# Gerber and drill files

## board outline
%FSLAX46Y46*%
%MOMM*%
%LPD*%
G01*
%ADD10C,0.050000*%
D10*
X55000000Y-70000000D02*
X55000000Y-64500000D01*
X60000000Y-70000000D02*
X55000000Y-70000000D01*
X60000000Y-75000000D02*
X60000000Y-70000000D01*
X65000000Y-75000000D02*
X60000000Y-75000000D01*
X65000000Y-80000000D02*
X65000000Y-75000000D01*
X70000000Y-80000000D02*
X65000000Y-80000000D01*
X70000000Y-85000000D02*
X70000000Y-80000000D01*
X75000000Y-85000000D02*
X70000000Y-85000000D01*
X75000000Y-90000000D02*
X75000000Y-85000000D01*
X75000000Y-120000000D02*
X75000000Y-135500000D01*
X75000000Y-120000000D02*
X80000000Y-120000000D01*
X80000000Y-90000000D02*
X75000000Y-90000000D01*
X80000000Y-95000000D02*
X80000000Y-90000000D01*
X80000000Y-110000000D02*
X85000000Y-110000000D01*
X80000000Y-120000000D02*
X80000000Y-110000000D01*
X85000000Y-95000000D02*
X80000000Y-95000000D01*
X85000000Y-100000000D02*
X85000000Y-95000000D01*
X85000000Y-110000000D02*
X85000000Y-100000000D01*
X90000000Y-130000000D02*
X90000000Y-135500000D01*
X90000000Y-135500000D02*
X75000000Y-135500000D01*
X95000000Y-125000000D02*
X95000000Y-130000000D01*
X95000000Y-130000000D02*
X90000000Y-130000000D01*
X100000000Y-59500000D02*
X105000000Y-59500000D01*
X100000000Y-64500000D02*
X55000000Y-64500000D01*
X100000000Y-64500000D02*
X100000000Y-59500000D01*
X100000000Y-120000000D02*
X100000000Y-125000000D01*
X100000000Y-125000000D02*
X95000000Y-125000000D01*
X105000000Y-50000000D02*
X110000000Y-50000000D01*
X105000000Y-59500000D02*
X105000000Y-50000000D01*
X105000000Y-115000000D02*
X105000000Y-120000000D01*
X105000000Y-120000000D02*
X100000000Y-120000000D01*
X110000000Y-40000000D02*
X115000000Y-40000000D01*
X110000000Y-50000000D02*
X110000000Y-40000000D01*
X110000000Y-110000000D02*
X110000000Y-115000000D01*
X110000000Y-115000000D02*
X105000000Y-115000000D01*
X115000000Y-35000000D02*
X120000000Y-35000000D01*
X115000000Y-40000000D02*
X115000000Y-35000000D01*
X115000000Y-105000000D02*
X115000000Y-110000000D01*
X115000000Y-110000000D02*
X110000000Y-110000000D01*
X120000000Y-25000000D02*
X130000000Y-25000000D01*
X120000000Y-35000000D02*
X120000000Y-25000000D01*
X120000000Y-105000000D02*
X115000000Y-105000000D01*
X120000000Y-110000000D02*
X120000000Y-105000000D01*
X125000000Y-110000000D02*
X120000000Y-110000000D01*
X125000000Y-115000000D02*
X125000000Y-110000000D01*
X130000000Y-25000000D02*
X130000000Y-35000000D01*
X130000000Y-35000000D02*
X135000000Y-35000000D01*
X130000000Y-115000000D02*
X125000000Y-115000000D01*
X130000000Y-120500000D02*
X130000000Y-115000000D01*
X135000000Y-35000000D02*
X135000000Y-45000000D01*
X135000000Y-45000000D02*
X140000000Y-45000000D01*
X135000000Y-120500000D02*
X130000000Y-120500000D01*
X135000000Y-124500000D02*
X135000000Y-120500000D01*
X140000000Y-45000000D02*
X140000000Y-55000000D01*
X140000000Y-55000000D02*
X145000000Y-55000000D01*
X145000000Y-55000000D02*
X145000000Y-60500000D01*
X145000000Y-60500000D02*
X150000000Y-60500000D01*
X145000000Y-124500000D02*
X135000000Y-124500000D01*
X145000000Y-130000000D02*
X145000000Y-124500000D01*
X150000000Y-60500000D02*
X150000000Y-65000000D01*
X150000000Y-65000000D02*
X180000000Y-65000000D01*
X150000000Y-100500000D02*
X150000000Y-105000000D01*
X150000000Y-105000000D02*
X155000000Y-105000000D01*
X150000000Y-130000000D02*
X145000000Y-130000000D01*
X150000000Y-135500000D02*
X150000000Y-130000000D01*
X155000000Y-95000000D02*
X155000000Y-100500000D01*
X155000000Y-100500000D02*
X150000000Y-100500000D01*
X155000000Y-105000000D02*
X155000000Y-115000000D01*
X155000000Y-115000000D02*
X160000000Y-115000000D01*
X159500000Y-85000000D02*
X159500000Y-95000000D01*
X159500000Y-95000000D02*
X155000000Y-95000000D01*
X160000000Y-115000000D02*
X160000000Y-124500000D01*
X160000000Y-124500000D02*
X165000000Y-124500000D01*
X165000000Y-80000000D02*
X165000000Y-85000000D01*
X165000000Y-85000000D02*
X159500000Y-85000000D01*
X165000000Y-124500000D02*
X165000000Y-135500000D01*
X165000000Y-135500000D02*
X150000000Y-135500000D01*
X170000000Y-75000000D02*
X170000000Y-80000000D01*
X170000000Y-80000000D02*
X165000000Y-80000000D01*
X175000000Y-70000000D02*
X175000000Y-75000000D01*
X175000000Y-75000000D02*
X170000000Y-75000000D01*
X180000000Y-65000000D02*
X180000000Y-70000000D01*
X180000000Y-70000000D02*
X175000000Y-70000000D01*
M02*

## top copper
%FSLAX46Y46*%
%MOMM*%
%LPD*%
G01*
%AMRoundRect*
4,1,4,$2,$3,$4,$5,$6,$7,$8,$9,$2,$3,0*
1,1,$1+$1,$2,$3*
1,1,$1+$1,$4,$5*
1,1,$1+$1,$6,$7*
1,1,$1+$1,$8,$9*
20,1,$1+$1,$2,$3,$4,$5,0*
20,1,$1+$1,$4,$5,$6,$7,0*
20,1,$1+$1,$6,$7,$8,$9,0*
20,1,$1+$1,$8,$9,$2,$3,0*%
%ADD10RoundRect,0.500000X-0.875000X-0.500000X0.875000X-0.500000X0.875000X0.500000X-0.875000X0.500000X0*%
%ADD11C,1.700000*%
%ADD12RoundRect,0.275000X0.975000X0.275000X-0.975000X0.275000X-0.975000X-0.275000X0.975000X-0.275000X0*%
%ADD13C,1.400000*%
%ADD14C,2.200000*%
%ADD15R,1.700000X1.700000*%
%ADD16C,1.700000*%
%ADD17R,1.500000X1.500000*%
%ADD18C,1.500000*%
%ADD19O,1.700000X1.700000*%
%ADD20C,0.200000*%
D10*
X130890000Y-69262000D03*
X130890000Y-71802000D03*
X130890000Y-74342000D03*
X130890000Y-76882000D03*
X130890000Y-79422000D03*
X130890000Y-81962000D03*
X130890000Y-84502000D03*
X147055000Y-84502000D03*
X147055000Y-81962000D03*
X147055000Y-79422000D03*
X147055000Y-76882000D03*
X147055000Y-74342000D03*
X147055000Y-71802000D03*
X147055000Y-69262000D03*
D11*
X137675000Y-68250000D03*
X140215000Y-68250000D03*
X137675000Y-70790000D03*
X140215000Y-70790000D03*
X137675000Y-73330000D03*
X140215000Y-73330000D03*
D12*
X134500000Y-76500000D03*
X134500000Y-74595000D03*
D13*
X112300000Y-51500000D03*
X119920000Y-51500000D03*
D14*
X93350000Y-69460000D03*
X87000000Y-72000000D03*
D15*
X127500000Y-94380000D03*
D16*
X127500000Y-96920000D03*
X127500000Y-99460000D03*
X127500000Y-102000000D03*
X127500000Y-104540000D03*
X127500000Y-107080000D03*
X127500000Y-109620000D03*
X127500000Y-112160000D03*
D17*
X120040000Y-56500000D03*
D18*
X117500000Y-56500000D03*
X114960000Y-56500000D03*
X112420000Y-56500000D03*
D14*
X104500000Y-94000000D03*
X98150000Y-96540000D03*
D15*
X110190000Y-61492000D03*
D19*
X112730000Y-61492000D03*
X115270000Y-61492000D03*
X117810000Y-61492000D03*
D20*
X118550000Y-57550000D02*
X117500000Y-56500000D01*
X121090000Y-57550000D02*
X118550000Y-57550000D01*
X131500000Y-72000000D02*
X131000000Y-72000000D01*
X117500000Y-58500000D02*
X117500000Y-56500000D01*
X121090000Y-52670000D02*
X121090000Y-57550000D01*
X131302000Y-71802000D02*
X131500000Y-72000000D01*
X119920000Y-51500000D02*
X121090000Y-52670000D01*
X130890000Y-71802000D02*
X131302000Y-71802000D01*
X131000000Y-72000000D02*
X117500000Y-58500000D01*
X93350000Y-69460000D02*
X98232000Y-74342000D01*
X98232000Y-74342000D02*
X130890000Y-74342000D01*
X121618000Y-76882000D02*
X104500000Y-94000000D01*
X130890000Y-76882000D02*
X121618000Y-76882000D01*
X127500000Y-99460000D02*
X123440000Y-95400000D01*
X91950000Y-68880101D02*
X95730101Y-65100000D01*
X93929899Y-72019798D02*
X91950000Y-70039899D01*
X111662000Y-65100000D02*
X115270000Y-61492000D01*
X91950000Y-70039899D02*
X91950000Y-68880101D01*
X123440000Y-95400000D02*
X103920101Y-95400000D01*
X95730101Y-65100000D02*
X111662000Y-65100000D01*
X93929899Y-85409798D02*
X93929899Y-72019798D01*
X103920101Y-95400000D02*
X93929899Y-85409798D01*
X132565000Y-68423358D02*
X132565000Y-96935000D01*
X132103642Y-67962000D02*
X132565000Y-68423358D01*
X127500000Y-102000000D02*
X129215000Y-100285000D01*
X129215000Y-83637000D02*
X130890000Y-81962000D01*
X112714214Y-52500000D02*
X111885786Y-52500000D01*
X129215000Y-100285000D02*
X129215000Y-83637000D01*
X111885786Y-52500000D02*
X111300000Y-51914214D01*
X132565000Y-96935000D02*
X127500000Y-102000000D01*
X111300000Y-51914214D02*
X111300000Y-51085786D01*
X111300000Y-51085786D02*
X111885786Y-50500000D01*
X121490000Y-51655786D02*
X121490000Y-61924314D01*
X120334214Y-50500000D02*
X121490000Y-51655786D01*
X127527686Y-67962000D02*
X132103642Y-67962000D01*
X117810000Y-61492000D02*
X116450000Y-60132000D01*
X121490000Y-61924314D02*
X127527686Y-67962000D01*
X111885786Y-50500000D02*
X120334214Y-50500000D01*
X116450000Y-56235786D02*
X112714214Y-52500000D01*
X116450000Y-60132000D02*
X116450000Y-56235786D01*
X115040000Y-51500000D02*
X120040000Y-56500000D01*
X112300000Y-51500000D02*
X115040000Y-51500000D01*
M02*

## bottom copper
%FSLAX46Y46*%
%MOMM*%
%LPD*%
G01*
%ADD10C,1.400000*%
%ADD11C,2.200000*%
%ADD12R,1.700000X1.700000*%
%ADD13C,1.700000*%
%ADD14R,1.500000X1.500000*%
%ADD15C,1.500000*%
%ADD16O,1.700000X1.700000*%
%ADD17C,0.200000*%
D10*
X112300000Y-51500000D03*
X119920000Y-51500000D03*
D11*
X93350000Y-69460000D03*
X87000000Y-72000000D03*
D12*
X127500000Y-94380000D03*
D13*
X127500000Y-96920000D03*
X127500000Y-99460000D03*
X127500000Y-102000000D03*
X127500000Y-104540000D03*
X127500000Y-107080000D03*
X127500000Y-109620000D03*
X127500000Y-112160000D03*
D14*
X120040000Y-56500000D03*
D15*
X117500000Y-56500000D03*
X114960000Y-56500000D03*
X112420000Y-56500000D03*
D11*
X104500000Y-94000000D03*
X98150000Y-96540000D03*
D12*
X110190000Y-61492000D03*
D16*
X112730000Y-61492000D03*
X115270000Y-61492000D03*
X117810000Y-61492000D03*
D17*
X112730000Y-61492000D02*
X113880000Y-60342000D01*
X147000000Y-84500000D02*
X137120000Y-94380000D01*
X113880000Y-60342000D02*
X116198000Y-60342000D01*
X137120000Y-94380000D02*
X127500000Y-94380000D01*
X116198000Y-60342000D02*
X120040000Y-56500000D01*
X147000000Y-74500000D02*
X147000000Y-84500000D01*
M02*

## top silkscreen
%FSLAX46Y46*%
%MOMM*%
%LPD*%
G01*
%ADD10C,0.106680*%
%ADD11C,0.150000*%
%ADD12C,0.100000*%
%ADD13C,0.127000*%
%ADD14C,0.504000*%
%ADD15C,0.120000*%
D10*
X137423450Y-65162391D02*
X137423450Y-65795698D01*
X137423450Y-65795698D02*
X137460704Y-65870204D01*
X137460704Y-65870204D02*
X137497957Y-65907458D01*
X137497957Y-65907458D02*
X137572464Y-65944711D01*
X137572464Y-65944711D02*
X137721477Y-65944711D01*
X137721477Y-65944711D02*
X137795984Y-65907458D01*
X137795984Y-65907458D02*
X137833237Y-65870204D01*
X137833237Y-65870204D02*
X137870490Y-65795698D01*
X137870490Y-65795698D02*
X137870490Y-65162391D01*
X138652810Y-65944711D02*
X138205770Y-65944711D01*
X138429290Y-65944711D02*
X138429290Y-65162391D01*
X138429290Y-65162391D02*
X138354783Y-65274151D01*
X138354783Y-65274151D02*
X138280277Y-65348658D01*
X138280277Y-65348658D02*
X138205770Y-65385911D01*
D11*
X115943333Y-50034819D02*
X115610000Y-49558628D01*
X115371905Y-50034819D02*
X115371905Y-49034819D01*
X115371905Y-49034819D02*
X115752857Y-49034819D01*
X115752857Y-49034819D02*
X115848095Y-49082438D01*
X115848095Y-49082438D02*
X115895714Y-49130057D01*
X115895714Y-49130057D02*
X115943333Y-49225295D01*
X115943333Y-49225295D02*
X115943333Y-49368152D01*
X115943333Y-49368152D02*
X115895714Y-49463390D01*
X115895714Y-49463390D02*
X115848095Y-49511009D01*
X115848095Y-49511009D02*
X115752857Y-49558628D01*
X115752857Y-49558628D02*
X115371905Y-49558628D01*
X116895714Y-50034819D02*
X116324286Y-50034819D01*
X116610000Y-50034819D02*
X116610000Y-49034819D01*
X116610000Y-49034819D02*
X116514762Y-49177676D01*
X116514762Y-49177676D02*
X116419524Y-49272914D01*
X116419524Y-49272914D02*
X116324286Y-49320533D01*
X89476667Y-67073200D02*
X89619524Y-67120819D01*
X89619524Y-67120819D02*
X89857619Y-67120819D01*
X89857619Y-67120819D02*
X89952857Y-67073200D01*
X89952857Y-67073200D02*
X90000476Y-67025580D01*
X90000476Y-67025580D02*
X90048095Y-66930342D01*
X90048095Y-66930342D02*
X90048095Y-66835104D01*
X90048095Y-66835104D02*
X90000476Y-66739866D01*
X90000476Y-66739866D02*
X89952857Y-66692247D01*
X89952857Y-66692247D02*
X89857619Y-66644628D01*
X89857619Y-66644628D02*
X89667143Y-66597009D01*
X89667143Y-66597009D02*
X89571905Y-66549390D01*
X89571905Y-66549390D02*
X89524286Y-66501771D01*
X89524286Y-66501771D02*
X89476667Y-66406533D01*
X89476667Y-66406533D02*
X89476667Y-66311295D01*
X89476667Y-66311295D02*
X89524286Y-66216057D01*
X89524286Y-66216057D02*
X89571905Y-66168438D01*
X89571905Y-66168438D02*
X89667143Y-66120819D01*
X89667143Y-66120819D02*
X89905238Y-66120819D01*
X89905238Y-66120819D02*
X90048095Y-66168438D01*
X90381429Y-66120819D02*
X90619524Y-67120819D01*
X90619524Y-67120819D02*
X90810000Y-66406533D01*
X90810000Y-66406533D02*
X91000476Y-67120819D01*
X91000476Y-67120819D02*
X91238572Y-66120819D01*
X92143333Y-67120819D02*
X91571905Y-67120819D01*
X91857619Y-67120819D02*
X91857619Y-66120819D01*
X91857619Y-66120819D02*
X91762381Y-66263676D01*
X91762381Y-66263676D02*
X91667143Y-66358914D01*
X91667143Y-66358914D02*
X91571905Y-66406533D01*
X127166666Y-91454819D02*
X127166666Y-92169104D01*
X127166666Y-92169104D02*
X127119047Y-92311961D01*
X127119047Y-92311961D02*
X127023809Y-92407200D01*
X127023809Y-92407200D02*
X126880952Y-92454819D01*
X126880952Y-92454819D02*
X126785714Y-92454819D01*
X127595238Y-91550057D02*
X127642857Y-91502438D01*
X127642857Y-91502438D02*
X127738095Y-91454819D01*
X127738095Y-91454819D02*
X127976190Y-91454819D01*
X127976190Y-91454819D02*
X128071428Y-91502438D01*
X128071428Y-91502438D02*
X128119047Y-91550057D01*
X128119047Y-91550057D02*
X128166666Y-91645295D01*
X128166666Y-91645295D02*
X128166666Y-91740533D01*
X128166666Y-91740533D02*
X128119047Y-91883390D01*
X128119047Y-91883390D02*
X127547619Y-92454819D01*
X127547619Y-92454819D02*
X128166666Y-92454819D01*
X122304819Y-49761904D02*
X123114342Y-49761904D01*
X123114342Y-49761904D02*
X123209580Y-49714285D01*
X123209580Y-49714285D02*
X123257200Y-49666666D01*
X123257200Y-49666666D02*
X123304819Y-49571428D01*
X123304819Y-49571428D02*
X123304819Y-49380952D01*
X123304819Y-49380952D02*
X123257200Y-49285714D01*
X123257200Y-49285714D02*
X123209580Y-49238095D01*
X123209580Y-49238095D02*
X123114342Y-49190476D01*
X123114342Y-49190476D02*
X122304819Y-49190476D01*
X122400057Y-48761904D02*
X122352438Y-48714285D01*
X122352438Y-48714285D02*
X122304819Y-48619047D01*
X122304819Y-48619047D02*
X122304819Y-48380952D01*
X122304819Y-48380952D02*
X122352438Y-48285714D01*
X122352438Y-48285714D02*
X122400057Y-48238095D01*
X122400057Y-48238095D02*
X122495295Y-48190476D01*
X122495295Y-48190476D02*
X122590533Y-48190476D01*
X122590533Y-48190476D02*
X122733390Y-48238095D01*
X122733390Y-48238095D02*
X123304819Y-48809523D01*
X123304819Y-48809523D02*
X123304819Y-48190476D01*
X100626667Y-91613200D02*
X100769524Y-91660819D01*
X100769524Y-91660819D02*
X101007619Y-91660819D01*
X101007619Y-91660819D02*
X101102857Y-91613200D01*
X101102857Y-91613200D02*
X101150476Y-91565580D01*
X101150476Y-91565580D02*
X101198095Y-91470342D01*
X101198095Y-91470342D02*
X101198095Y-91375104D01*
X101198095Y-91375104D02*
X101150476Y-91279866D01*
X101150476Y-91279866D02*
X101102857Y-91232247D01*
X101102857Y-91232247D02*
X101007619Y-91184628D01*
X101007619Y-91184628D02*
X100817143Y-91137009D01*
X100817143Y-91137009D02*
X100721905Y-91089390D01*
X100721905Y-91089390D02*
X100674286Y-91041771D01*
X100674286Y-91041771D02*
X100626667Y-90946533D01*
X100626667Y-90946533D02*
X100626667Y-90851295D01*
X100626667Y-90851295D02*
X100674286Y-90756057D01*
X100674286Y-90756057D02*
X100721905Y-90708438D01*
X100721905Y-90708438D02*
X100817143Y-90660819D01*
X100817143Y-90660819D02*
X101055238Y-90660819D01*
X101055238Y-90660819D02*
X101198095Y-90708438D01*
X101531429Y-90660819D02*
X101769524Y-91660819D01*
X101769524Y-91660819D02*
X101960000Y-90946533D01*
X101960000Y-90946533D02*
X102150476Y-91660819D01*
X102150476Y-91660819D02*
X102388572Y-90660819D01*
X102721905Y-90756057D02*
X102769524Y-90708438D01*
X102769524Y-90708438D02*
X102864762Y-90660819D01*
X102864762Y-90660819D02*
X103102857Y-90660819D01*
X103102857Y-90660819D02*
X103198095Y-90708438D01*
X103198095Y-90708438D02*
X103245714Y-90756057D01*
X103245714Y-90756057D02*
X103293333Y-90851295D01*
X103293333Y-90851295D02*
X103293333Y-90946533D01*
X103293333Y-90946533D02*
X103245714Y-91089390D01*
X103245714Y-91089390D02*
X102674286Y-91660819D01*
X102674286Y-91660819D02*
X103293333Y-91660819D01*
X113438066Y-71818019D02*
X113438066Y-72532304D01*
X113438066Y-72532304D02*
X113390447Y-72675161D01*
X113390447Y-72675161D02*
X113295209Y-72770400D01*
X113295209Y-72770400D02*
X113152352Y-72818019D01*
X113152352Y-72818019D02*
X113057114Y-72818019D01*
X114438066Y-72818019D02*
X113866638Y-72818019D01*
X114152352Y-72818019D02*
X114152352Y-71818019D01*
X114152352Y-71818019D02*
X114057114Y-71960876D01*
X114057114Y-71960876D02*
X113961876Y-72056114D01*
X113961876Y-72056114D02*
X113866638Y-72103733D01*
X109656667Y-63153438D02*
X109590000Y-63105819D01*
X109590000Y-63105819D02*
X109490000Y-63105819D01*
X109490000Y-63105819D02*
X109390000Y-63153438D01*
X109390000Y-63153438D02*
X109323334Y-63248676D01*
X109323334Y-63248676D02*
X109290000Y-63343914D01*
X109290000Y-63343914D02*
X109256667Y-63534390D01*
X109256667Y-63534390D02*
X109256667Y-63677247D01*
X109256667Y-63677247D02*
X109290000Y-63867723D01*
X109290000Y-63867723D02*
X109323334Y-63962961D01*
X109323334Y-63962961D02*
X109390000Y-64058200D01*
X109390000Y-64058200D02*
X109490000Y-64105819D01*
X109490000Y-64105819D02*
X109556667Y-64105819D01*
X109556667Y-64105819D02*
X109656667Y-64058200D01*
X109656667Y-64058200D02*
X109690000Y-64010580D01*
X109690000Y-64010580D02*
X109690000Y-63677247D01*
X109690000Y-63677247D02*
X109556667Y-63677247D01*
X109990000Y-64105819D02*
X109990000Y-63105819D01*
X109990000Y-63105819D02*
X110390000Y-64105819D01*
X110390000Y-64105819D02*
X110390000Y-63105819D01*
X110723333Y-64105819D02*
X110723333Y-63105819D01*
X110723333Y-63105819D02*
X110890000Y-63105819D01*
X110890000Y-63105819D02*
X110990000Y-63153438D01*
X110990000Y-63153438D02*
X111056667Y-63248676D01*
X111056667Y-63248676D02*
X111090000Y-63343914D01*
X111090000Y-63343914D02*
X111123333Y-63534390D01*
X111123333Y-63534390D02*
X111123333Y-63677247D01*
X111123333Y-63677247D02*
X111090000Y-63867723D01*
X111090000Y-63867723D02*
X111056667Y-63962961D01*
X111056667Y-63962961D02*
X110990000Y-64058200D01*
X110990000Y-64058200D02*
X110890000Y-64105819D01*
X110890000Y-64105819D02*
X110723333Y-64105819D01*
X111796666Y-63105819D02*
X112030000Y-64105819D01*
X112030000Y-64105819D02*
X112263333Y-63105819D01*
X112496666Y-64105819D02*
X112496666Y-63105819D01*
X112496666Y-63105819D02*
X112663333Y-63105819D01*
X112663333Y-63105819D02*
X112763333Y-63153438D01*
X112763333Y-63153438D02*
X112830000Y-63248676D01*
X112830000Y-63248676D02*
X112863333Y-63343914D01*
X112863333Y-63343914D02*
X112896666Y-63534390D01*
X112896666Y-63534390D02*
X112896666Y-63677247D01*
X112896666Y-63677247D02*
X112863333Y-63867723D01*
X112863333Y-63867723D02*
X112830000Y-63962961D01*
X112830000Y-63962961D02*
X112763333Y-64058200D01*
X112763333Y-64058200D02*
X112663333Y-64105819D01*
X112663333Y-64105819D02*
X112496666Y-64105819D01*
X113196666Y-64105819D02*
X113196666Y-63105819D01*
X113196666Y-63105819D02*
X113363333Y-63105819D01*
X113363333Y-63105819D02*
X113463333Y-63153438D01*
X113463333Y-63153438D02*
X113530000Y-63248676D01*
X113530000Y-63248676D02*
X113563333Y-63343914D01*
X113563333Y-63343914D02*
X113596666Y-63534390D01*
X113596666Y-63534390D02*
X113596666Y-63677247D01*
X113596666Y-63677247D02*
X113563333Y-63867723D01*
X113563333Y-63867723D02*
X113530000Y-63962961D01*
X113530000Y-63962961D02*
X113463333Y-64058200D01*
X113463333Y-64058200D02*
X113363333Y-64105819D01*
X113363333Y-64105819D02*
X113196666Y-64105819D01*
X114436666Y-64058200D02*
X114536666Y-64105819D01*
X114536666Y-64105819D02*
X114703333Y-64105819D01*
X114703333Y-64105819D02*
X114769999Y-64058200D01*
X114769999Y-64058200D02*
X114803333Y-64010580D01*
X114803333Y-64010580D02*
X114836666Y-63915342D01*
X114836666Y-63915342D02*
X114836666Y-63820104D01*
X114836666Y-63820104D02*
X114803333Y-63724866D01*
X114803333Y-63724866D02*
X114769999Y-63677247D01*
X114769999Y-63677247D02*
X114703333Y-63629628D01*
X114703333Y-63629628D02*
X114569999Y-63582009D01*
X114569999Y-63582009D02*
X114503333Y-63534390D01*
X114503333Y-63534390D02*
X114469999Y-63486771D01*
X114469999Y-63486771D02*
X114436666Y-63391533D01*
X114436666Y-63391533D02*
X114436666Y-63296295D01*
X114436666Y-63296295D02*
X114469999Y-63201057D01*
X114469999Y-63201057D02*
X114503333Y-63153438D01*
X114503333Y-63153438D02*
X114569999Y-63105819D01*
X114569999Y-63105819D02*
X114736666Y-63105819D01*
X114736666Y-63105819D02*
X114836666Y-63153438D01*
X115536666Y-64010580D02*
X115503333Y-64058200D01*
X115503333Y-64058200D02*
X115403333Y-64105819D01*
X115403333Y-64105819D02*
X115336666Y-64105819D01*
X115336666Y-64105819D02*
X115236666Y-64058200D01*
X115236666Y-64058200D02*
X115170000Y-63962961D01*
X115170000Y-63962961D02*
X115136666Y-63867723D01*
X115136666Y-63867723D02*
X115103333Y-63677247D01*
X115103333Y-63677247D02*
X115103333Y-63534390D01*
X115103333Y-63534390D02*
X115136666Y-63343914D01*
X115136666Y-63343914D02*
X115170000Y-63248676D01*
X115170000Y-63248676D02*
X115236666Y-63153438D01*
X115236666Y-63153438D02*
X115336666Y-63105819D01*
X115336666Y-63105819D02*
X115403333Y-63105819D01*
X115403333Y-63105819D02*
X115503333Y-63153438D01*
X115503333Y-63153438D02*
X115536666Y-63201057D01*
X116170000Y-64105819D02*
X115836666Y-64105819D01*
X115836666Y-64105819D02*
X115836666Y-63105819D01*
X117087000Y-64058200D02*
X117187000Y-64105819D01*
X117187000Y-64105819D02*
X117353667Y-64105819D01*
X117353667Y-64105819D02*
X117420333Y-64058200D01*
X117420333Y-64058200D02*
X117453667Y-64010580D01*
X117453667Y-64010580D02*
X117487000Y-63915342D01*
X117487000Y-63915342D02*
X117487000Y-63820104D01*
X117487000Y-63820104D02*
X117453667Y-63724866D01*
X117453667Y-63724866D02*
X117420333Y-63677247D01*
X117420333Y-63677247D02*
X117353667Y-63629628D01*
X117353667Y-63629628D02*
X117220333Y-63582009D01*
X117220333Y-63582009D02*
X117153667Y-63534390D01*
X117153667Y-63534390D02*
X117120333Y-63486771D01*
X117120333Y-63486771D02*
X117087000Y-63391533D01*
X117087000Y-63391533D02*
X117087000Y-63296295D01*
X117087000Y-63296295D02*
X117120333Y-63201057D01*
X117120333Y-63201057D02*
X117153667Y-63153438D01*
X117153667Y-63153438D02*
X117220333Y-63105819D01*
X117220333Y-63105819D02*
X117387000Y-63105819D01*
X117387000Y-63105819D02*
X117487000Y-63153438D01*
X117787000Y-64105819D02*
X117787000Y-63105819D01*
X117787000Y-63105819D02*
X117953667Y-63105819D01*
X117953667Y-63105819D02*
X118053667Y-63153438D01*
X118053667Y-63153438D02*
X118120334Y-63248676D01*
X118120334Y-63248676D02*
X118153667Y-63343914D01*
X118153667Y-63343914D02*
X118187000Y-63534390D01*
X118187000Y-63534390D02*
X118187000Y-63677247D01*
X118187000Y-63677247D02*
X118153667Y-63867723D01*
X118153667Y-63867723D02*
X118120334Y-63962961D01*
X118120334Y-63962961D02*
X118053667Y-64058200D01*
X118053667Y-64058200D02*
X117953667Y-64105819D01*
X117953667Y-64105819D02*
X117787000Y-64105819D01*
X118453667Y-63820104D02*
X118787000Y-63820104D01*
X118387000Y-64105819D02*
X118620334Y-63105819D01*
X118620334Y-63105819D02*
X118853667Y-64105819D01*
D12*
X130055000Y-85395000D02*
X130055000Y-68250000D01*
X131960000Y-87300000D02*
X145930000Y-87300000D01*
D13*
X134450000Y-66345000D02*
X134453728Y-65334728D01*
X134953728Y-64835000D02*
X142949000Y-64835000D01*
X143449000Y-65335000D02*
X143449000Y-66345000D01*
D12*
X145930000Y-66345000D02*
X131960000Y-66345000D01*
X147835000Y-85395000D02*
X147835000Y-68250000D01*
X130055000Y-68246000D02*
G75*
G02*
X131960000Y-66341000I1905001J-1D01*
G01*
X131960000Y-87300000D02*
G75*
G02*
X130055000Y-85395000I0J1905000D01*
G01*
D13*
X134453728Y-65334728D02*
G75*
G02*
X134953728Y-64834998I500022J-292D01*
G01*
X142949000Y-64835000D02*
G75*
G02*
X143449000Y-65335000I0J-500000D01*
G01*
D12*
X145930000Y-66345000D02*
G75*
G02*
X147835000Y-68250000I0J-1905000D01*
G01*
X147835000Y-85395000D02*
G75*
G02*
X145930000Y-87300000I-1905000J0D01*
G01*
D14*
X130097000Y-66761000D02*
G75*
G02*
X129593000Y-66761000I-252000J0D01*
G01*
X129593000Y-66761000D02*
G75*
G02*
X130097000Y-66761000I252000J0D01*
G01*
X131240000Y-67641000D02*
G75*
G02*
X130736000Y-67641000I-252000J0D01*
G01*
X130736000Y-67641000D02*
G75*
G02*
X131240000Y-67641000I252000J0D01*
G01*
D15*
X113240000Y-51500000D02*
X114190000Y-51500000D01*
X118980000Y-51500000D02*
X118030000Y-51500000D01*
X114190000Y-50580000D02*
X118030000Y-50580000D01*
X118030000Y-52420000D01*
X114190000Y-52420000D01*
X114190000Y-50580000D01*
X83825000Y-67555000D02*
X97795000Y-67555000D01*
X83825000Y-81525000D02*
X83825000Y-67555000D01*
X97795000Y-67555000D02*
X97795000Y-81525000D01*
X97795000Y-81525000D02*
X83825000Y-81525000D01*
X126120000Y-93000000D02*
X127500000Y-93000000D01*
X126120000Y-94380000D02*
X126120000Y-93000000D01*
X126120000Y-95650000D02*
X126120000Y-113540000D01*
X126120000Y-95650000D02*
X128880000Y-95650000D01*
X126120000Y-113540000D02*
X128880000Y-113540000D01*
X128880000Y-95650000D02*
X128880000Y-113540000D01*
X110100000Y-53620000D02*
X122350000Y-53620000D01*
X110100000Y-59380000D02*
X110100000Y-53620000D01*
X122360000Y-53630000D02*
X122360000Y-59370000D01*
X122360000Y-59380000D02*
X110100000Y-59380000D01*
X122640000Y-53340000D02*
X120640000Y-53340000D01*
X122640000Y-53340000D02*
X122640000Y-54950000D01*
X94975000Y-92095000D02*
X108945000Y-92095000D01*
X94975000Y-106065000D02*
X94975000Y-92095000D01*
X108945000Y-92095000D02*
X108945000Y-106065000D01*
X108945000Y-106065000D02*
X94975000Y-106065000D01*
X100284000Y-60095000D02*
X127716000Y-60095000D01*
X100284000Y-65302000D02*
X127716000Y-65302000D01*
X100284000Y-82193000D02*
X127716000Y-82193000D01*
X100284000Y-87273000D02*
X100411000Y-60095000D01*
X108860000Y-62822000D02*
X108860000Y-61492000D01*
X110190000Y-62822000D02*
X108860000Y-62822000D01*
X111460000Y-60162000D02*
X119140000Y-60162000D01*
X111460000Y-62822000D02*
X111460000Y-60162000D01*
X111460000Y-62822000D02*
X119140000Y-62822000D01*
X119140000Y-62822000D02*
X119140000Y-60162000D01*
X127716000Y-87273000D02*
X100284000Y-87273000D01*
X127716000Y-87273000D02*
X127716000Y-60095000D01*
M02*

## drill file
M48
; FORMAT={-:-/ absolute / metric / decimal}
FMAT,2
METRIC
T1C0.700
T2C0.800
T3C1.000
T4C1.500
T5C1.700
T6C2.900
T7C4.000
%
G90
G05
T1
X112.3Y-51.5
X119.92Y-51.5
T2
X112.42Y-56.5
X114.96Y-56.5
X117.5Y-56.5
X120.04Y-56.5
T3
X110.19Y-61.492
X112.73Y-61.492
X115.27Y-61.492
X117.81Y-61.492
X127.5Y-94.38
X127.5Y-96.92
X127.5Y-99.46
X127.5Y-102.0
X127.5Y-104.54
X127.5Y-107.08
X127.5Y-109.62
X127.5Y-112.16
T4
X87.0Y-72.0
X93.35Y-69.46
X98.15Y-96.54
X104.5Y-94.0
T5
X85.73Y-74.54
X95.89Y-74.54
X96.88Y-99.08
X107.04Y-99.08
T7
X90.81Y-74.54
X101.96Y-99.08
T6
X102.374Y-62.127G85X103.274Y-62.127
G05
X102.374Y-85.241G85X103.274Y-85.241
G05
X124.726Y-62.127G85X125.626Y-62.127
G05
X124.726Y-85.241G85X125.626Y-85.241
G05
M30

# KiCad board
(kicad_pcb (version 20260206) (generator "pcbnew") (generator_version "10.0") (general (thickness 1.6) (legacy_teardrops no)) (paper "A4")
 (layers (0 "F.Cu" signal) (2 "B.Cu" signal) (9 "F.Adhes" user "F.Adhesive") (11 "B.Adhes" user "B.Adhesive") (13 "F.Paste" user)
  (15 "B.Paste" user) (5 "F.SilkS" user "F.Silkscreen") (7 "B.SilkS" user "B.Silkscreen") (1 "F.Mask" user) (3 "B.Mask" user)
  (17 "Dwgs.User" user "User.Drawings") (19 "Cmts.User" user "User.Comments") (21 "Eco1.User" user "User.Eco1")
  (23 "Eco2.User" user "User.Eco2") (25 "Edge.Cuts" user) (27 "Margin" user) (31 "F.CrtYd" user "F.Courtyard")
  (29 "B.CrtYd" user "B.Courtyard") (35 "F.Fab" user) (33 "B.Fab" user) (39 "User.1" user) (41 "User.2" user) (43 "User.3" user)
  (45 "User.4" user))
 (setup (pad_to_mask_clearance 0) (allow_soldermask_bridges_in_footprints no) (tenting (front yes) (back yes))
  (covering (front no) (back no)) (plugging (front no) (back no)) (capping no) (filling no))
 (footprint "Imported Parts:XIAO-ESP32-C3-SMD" (layer "F.Cu") (at 130.055 87.382)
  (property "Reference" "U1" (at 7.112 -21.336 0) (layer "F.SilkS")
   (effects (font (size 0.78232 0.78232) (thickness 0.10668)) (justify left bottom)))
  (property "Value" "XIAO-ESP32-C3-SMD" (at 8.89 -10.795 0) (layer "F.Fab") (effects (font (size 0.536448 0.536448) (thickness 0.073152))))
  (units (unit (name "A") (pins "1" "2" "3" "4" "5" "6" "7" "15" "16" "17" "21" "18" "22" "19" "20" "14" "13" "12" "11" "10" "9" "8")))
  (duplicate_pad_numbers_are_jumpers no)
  (fp_line (start 0 -1.987) (end 0 -19.132) (stroke (width 0.1) (type solid)) (layer "F.SilkS"))
  (fp_line (start 1.905 -0.082) (end 15.875 -0.082) (stroke (width 0.1) (type solid)) (layer "F.SilkS"))
  (fp_line (start 4.395 -21.037) (end 4.398728 -22.047272) (stroke (width 0.127) (type solid)) (layer "F.SilkS"))
  (fp_line (start 4.898728 -22.547) (end 12.894 -22.547) (stroke (width 0.127) (type solid)) (layer "F.SilkS"))
  (fp_line (start 13.394 -22.047) (end 13.394 -21.037) (stroke (width 0.127) (type solid)) (layer "F.SilkS"))
  (fp_line (start 15.875 -21.037) (end 1.905 -21.037) (stroke (width 0.1) (type solid)) (layer "F.SilkS"))
  (fp_line (start 17.78 -1.987) (end 17.78 -19.132) (stroke (width 0.1) (type solid)) (layer "F.SilkS"))
  (fp_arc (start 0 -19.136) (mid 0.557962 -20.483038) (end 1.905 -21.041) (stroke (width 0.1) (type solid)) (layer "F.SilkS"))
  (fp_arc (start 1.905 -0.082) (mid 0.557962 -0.639962) (end 0 -1.987) (stroke (width 0.1) (type solid)) (layer "F.SilkS"))
  (fp_arc (start 4.398728 -22.047272) (mid 4.545272 -22.40064) (end 4.898728 -22.547) (stroke (width 0.127) (type default))
   (layer "F.SilkS"))
  (fp_arc (start 12.894 -22.547) (mid 13.247553 -22.400553) (end 13.394 -22.047) (stroke (width 0.127) (type default)) (layer "F.SilkS"))
  (fp_arc (start 15.875 -21.037) (mid 17.222038 -20.479038) (end 17.78 -19.132) (stroke (width 0.1) (type solid)) (layer "F.SilkS"))
  (fp_arc (start 17.78 -1.987) (mid 17.222038 -0.639962) (end 15.875 -0.082) (stroke (width 0.1) (type solid)) (layer "F.SilkS"))
  (fp_circle (center -0.21 -20.621) (end -0.21 -20.875) (stroke (width 0.5) (type solid)) (fill yes) (layer "F.SilkS"))
  (fp_circle (center 0.933 -19.741) (end 0.933 -19.995) (stroke (width 0.5) (type solid)) (fill yes) (layer "F.SilkS"))
  (pad "1" smd roundrect (at 0.835 -18.12) (size 2.75 2) (layers "F.Cu" "F.Mask" "F.Paste") (roundrect_rratio 0.25)
   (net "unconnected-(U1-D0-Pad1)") (solder_mask_margin 0.0508) (thermal_bridge_angle 45))
  (pad "2" smd roundrect (at 0.835 -15.58) (size 2.75 2) (layers "F.Cu" "F.Mask" "F.Paste") (roundrect_rratio 0.25) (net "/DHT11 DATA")
   (solder_mask_margin 0.0508) (thermal_bridge_angle 45))
  (pad "3" smd roundrect (at 0.835 -13.04) (size 2.75 2) (layers "F.Cu" "F.Mask" "F.Paste") (roundrect_rratio 0.25) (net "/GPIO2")
   (solder_mask_margin 0.0508) (thermal_bridge_angle 45))
  (pad "4" smd roundrect (at 0.835 -10.5) (size 2.75 2) (layers "F.Cu" "F.Mask" "F.Paste") (roundrect_rratio 0.25) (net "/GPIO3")
   (solder_mask_margin 0.0508) (thermal_bridge_angle 45))
  (pad "5" smd roundrect (at 0.835 -7.96) (size 2.75 2) (layers "F.Cu" "F.Mask" "F.Paste") (roundrect_rratio 0.25) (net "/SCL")
   (solder_mask_margin 0.0508) (thermal_bridge_angle 45))
  (pad "6" smd roundrect (at 0.835 -5.42) (size 2.75 2) (layers "F.Cu" "F.Mask" "F.Paste") (roundrect_rratio 0.25) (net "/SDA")
   (solder_mask_margin 0.0508) (thermal_bridge_angle 45))
  (pad "7" smd roundrect (at 0.835 -2.88) (size 2.75 2) (layers "F.Cu" "F.Mask" "F.Paste") (roundrect_rratio 0.25)
   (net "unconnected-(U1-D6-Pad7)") (solder_mask_margin 0.0508) (thermal_bridge_angle 45))
  (pad "8" smd roundrect (at 17 -2.88) (size 2.75 2) (layers "F.Cu" "F.Mask" "F.Paste") (roundrect_rratio 0.25)
   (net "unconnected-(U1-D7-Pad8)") (solder_mask_margin 0.0508) (thermal_bridge_angle 45))
  (pad "9" smd roundrect (at 17 -5.42) (size 2.75 2) (layers "F.Cu" "F.Mask" "F.Paste") (roundrect_rratio 0.25)
   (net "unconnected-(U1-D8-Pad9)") (solder_mask_margin 0.0508) (thermal_bridge_angle 45))
  (pad "10" smd roundrect (at 17 -7.96) (size 2.75 2) (layers "F.Cu" "F.Mask" "F.Paste") (roundrect_rratio 0.25)
   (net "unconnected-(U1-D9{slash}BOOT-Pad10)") (solder_mask_margin 0.0508) (thermal_bridge_angle 45))
  (pad "11" smd roundrect (at 17 -10.5) (size 2.75 2) (layers "F.Cu" "F.Mask" "F.Paste") (roundrect_rratio 0.25)
   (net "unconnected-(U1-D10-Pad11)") (solder_mask_margin 0.0508) (thermal_bridge_angle 45))
  (pad "12" smd roundrect (at 17 -13.04) (size 2.75 2) (layers "F.Cu" "F.Mask" "F.Paste") (roundrect_rratio 0.25) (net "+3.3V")
   (solder_mask_margin 0.0508) (thermal_bridge_angle 45))
  (pad "13" smd roundrect (at 17 -15.58) (size 2.75 2) (layers "F.Cu" "F.Mask" "F.Paste") (roundrect_rratio 0.25) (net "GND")
   (solder_mask_margin 0.0508) (thermal_bridge_angle 45))
  (pad "14" smd roundrect (at 17 -18.12) (size 2.75 2) (layers "F.Cu" "F.Mask" "F.Paste") (roundrect_rratio 0.25) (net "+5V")
   (solder_mask_margin 0.0508) (thermal_bridge_angle 45))
  (pad "15" smd circle (at 7.62 -19.132) (size 1.7 1.7) (layers "F.Cu" "F.Mask" "F.Paste") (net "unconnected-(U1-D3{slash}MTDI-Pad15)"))
  (pad "16" smd circle (at 10.16 -19.132) (size 1.7 1.7) (layers "F.Cu" "F.Mask" "F.Paste") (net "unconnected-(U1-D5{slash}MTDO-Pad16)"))
  (pad "17" smd circle (at 7.62 -16.592) (size 1.7 1.7) (layers "F.Cu" "F.Mask" "F.Paste") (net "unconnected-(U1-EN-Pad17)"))
  (pad "18" smd circle (at 10.16 -16.592) (size 1.7 1.7) (layers "F.Cu" "F.Mask" "F.Paste") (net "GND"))
  (pad "19" smd circle (at 7.62 -14.052) (size 1.7 1.7) (layers "F.Cu" "F.Mask" "F.Paste") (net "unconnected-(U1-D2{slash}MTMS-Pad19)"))
  (pad "20" smd circle (at 10.16 -14.052) (size 1.7 1.7) (layers "F.Cu" "F.Mask" "F.Paste") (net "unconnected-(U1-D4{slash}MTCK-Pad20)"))
  (pad "21" smd roundrect (at 4.445 -10.882 180) (size 2.5 1.1) (layers "F.Cu" "F.Mask" "F.Paste") (roundrect_rratio 0.25)
   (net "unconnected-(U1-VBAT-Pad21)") (thermal_bridge_angle 45))
  (pad "22" smd roundrect (at 4.445 -12.787 180) (size 2.5 1.1) (layers "F.Cu" "F.Mask" "F.Paste") (roundrect_rratio 0.25)
   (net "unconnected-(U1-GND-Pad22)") (thermal_bridge_angle 45)))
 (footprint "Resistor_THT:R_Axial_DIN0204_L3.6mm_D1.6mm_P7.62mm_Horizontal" (layer "F.Cu") (at 112.3 51.5)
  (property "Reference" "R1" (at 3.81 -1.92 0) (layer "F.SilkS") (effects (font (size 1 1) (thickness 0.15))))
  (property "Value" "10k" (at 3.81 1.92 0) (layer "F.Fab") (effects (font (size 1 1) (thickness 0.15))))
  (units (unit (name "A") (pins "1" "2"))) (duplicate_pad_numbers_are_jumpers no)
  (fp_line (start 0.94 0) (end 1.89 0) (stroke (width 0.12) (type solid)) (layer "F.SilkS"))
  (fp_line (start 6.68 0) (end 5.73 0) (stroke (width 0.12) (type solid)) (layer "F.SilkS"))
  (fp_rect (start 1.89 -0.92) (end 5.73 0.92) (stroke (width 0.12) (type solid)) (fill no) (layer "F.SilkS"))
  (pad "1" thru_hole circle (at 0 0) (size 1.4 1.4) (drill 0.7) (layers "*.Cu" "*.Mask") (remove_unused_layers no) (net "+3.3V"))
  (pad "2" thru_hole circle (at 7.62 0) (size 1.4 1.4) (drill 0.7) (layers "*.Cu" "*.Mask") (remove_unused_layers no) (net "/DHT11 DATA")))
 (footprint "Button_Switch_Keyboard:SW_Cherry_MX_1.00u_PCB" (layer "F.Cu") (at 93.35 69.46)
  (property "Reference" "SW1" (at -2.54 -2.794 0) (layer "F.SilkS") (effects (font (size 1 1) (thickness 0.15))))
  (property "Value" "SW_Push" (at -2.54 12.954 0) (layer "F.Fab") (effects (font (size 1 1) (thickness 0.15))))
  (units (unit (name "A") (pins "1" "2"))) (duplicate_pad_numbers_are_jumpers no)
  (fp_line (start -9.525 -1.905) (end 4.445 -1.905) (stroke (width 0.12) (type solid)) (layer "F.SilkS"))
  (fp_line (start -9.525 12.065) (end -9.525 -1.905) (stroke (width 0.12) (type solid)) (layer "F.SilkS"))
  (fp_line (start 4.445 -1.905) (end 4.445 12.065) (stroke (width 0.12) (type solid)) (layer "F.SilkS"))
  (fp_line (start 4.445 12.065) (end -9.525 12.065) (stroke (width 0.12) (type solid)) (layer "F.SilkS"))
  (pad "" np_thru_hole circle (at -7.62 5.08) (size 1.7 1.7) (drill 1.7) (layers "*.Cu" "*.Mask"))
  (pad "" np_thru_hole circle (at -2.54 5.08) (size 4 4) (drill 4) (layers "*.Cu" "*.Mask"))
  (pad "" np_thru_hole circle (at 2.54 5.08) (size 1.7 1.7) (drill 1.7) (layers "*.Cu" "*.Mask"))
  (pad "1" thru_hole circle (at 0 0) (size 2.2 2.2) (drill 1.5) (layers "*.Cu" "*.Mask") (remove_unused_layers no) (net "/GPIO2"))
  (pad "2" thru_hole circle (at -6.35 2.54) (size 2.2 2.2) (drill 1.5) (layers "*.Cu" "*.Mask") (remove_unused_layers no) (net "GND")))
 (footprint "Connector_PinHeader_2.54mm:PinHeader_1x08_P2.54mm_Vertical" (layer "F.Cu") (at 127.5 94.38)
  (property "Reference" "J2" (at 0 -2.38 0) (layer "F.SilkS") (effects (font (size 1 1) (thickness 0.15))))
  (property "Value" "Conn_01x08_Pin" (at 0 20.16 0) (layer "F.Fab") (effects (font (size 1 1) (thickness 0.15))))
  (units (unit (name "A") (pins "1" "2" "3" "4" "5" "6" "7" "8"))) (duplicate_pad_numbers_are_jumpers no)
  (fp_line (start -1.38 -1.38) (end 0 -1.38) (stroke (width 0.12) (type solid)) (layer "F.SilkS"))
  (fp_line (start -1.38 0) (end -1.38 -1.38) (stroke (width 0.12) (type solid)) (layer "F.SilkS"))
  (fp_line (start -1.38 1.27) (end -1.38 19.16) (stroke (width 0.12) (type solid)) (layer "F.SilkS"))
  (fp_line (start -1.38 1.27) (end 1.38 1.27) (stroke (width 0.12) (type solid)) (layer "F.SilkS"))
  (fp_line (start -1.38 19.16) (end 1.38 19.16) (stroke (width 0.12) (type solid)) (layer "F.SilkS"))
  (fp_line (start 1.38 1.27) (end 1.38 19.16) (stroke (width 0.12) (type solid)) (layer "F.SilkS"))
  (pad "1" thru_hole rect (at 0 0) (size 1.7 1.7) (drill 1) (layers "*.Cu" "*.Mask") (remove_unused_layers no) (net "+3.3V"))
  (pad "2" thru_hole circle (at 0 2.54) (size 1.7 1.7) (drill 1) (layers "*.Cu" "*.Mask") (remove_unused_layers no) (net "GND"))
  (pad "3" thru_hole circle (at 0 5.08) (size 1.7 1.7) (drill 1) (layers "*.Cu" "*.Mask") (remove_unused_layers no) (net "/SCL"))
  (pad "4" thru_hole circle (at 0 7.62) (size 1.7 1.7) (drill 1) (layers "*.Cu" "*.Mask") (remove_unused_layers no) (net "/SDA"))
  (pad "5" thru_hole circle (at 0 10.16) (size 1.7 1.7) (drill 1) (layers "*.Cu" "*.Mask") (remove_unused_layers no)
   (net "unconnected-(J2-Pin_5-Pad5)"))
  (pad "6" thru_hole circle (at 0 12.7) (size 1.7 1.7) (drill 1) (layers "*.Cu" "*.Mask") (remove_unused_layers no)
   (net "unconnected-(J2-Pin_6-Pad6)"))
  (pad "7" thru_hole circle (at 0 15.24) (size 1.7 1.7) (drill 1) (layers "*.Cu" "*.Mask") (remove_unused_layers no)
   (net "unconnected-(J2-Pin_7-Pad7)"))
  (pad "8" thru_hole circle (at 0 17.78) (size 1.7 1.7) (drill 1) (layers "*.Cu" "*.Mask") (remove_unused_layers no)
   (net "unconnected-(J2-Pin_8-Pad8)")))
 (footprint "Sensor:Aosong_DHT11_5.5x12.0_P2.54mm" (layer "F.Cu") (at 120.04 56.5 -90)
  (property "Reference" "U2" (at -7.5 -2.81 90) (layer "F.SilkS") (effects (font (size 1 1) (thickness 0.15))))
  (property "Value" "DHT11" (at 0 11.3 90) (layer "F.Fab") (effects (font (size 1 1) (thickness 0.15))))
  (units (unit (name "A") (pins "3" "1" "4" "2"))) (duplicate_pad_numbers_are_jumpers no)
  (fp_line (start -2.88 9.94) (end -2.88 -2.31) (stroke (width 0.12) (type solid)) (layer "F.SilkS"))
  (fp_line (start 2.88 9.94) (end -2.88 9.94) (stroke (width 0.12) (type solid)) (layer "F.SilkS"))
  (fp_line (start -2.87 -2.32) (end 2.87 -2.32) (stroke (width 0.12) (type solid)) (layer "F.SilkS"))
  (fp_line (start 2.88 -2.32) (end 2.88 9.94) (stroke (width 0.12) (type solid)) (layer "F.SilkS"))
  (fp_line (start -3.16 -2.6) (end -3.16 -0.6) (stroke (width 0.12) (type solid)) (layer "F.SilkS"))
  (fp_line (start -3.16 -2.6) (end -1.55 -2.6) (stroke (width 0.12) (type solid)) (layer "F.SilkS"))
  (pad "1" thru_hole rect (at 0 0 270) (size 1.5 1.5) (drill 0.8) (layers "*.Cu" "*.Mask") (remove_unused_layers no) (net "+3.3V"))
  (pad "2" thru_hole circle (at 0 2.54 270) (size 1.5 1.5) (drill 0.8) (layers "*.Cu" "*.Mask") (remove_unused_layers no)
   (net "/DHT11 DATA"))
  (pad "3" thru_hole circle (at 0 5.08 270) (size 1.5 1.5) (drill 0.8) (layers "*.Cu" "*.Mask") (remove_unused_layers no)
   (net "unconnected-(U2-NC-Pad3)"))
  (pad "4" thru_hole circle (at 0 7.62 270) (size 1.5 1.5) (drill 0.8) (layers "*.Cu" "*.Mask") (remove_unused_layers no) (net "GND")))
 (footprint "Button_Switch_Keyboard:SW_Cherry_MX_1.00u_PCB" (layer "F.Cu") (at 104.5 94)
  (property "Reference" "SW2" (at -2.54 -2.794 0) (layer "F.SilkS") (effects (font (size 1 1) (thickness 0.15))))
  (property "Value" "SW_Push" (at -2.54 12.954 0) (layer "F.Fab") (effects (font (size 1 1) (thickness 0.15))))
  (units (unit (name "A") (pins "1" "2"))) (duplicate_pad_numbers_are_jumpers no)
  (fp_line (start -9.525 -1.905) (end 4.445 -1.905) (stroke (width 0.12) (type solid)) (layer "F.SilkS"))
  (fp_line (start -9.525 12.065) (end -9.525 -1.905) (stroke (width 0.12) (type solid)) (layer "F.SilkS"))
  (fp_line (start 4.445 -1.905) (end 4.445 12.065) (stroke (width 0.12) (type solid)) (layer "F.SilkS"))
  (fp_line (start 4.445 12.065) (end -9.525 12.065) (stroke (width 0.12) (type solid)) (layer "F.SilkS"))
  (pad "" np_thru_hole circle (at -7.62 5.08) (size 1.7 1.7) (drill 1.7) (layers "*.Cu" "*.Mask"))
  (pad "" np_thru_hole circle (at -2.54 5.08) (size 4 4) (drill 4) (layers "*.Cu" "*.Mask"))
  (pad "" np_thru_hole circle (at 2.54 5.08) (size 1.7 1.7) (drill 1.7) (layers "*.Cu" "*.Mask"))
  (pad "1" thru_hole circle (at 0 0) (size 2.2 2.2) (drill 1.5) (layers "*.Cu" "*.Mask") (remove_unused_layers no) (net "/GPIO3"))
  (pad "2" thru_hole circle (at -6.35 2.54) (size 2.2 2.2) (drill 1.5) (layers "*.Cu" "*.Mask") (remove_unused_layers no) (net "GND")))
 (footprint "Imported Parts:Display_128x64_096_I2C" (layer "F.Cu") (at 114 61.492)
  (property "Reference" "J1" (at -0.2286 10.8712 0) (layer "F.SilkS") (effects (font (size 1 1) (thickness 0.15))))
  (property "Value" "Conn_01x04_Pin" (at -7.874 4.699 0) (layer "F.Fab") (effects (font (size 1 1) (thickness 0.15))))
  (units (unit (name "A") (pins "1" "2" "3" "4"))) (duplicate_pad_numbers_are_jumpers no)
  (fp_line (start -13.716 -1.397) (end 13.716 -1.397) (stroke (width 0.12) (type solid)) (layer "F.SilkS"))
  (fp_line (start -13.716 3.81) (end 13.716 3.81) (stroke (width 0.12) (type solid)) (layer "F.SilkS"))
  (fp_line (start -13.716 20.701) (end 13.716 20.701) (stroke (width 0.12) (type solid)) (layer "F.SilkS"))
  (fp_line (start -13.716 25.781) (end -13.589 -1.397) (stroke (width 0.12) (type solid)) (layer "F.SilkS"))
  (fp_line (start -5.14 1.33) (end -5.14 0) (stroke (width 0.12) (type solid)) (layer "F.SilkS"))
  (fp_line (start -3.81 1.33) (end -5.14 1.33) (stroke (width 0.12) (type solid)) (layer "F.SilkS"))
  (fp_line (start -2.54 -1.33) (end 5.14 -1.33) (stroke (width 0.12) (type solid)) (layer "F.SilkS"))
  (fp_line (start -2.54 1.33) (end -2.54 -1.33) (stroke (width 0.12) (type solid)) (layer "F.SilkS"))
  (fp_line (start -2.54 1.33) (end 5.14 1.33) (stroke (width 0.12) (type solid)) (layer "F.SilkS"))
  (fp_line (start 5.14 1.33) (end 5.14 -1.33) (stroke (width 0.12) (type solid)) (layer "F.SilkS"))
  (fp_line (start 13.716 25.781) (end -13.716 25.781) (stroke (width 0.12) (type solid)) (layer "F.SilkS"))
  (fp_line (start 13.716 25.781) (end 13.716 -1.397) (stroke (width 0.12) (type solid)) (layer "F.SilkS"))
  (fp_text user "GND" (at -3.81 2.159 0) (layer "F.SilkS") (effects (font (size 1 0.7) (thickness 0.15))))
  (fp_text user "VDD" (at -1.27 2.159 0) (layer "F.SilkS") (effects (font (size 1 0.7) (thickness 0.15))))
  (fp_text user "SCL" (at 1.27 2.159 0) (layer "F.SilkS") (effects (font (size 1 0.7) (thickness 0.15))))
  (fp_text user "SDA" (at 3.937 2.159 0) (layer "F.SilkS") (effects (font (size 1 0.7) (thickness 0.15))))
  (pad "" np_thru_hole oval (at -11.176 0.635) (size 3.8 2.9) (drill oval 3.8 2.9) (layers "*.Cu" "*.Mask"))
  (pad "" np_thru_hole oval (at -11.176 23.749) (size 3.8 2.9) (drill oval 3.8 2.9) (layers "*.Cu" "*.Mask"))
  (pad "" np_thru_hole oval (at 11.176 0.635) (size 3.8 2.9) (drill oval 3.8 2.9) (layers "*.Cu" "*.Mask"))
  (pad "" np_thru_hole oval (at 11.176 23.749) (size 3.8 2.9) (drill oval 3.8 2.9) (layers "*.Cu" "*.Mask"))
  (pad "1" thru_hole rect (at -3.81 0 90) (size 1.7 1.7) (drill 1) (layers "*.Cu" "*.Mask") (remove_unused_layers no) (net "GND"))
  (pad "2" thru_hole oval (at -1.27 0 90) (size 1.7 1.7) (drill 1) (layers "*.Cu" "*.Mask") (remove_unused_layers no) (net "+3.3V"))
  (pad "3" thru_hole oval (at 1.27 0 90) (size 1.7 1.7) (drill 1) (layers "*.Cu" "*.Mask") (remove_unused_layers no) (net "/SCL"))
  (pad "4" thru_hole oval (at 3.81 0 90) (size 1.7 1.7) (drill 1) (layers "*.Cu" "*.Mask") (remove_unused_layers no) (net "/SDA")))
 (gr_line (start 55 70) (end 55 64.5) (stroke (width 0.05) (type default)) (layer "Edge.Cuts"))
 (gr_line (start 60 70) (end 55 70) (stroke (width 0.05) (type default)) (layer "Edge.Cuts"))
 (gr_line (start 60 75) (end 60 70) (stroke (width 0.05) (type default)) (layer "Edge.Cuts"))
 (gr_line (start 65 75) (end 60 75) (stroke (width 0.05) (type default)) (layer "Edge.Cuts"))
 (gr_line (start 65 80) (end 65 75) (stroke (width 0.05) (type default)) (layer "Edge.Cuts"))
 (gr_line (start 70 80) (end 65 80) (stroke (width 0.05) (type default)) (layer "Edge.Cuts"))
 (gr_line (start 70 85) (end 70 80) (stroke (width 0.05) (type default)) (layer "Edge.Cuts"))
 (gr_line (start 75 85) (end 70 85) (stroke (width 0.05) (type default)) (layer "Edge.Cuts"))
 (gr_line (start 75 90) (end 75 85) (stroke (width 0.05) (type default)) (layer "Edge.Cuts"))
 (gr_line (start 75 120) (end 75 135.5) (stroke (width 0.05) (type default)) (layer "Edge.Cuts"))
 (gr_line (start 75 120) (end 80 120) (stroke (width 0.05) (type default)) (layer "Edge.Cuts"))
 (gr_line (start 80 90) (end 75 90) (stroke (width 0.05) (type default)) (layer "Edge.Cuts"))
 (gr_line (start 80 95) (end 80 90) (stroke (width 0.05) (type default)) (layer "Edge.Cuts"))
 (gr_line (start 80 110) (end 85 110) (stroke (width 0.05) (type default)) (layer "Edge.Cuts"))
 (gr_line (start 80 120) (end 80 110) (stroke (width 0.05) (type default)) (layer "Edge.Cuts"))
 (gr_line (start 85 95) (end 80 95) (stroke (width 0.05) (type default)) (layer "Edge.Cuts"))
 (gr_line (start 85 100) (end 85 95) (stroke (width 0.05) (type default)) (layer "Edge.Cuts"))
 (gr_line (start 85 110) (end 85 100) (stroke (width 0.05) (type default)) (layer "Edge.Cuts"))
 (gr_line (start 90 130) (end 90 135.5) (stroke (width 0.05) (type default)) (layer "Edge.Cuts"))
 (gr_line (start 90 135.5) (end 75 135.5) (stroke (width 0.05) (type default)) (layer "Edge.Cuts"))
 (gr_line (start 95 125) (end 95 130) (stroke (width 0.05) (type default)) (layer "Edge.Cuts"))
 (gr_line (start 95 130) (end 90 130) (stroke (width 0.05) (type default)) (layer "Edge.Cuts"))
 (gr_line (start 100 59.5) (end 105 59.5) (stroke (width 0.05) (type default)) (layer "Edge.Cuts"))
 (gr_line (start 100 64.5) (end 55 64.5) (stroke (width 0.05) (type default)) (layer "Edge.Cuts"))
 (gr_line (start 100 64.5) (end 100 59.5) (stroke (width 0.05) (type default)) (layer "Edge.Cuts"))
 (gr_line (start 100 120) (end 100 125) (stroke (width 0.05) (type default)) (layer "Edge.Cuts"))
 (gr_line (start 100 125) (end 95 125) (stroke (width 0.05) (type default)) (layer "Edge.Cuts"))
 (gr_line (start 105 50) (end 110 50) (stroke (width 0.05) (type default)) (layer "Edge.Cuts"))
 (gr_line (start 105 59.5) (end 105 50) (stroke (width 0.05) (type default)) (layer "Edge.Cuts"))
 (gr_line (start 105 115) (end 105 120) (stroke (width 0.05) (type default)) (layer "Edge.Cuts"))
 (gr_line (start 105 120) (end 100 120) (stroke (width 0.05) (type default)) (layer "Edge.Cuts"))
 (gr_line (start 110 40) (end 115 40) (stroke (width 0.05) (type default)) (layer "Edge.Cuts"))
 (gr_line (start 110 50) (end 110 40) (stroke (width 0.05) (type default)) (layer "Edge.Cuts"))
 (gr_line (start 110 110) (end 110 115) (stroke (width 0.05) (type default)) (layer "Edge.Cuts"))
 (gr_line (start 110 115) (end 105 115) (stroke (width 0.05) (type default)) (layer "Edge.Cuts"))
 (gr_line (start 115 35) (end 120 35) (stroke (width 0.05) (type default)) (layer "Edge.Cuts"))
 (gr_line (start 115 40) (end 115 35) (stroke (width 0.05) (type default)) (layer "Edge.Cuts"))
 (gr_line (start 115 105) (end 115 110) (stroke (width 0.05) (type default)) (layer "Edge.Cuts"))
 (gr_line (start 115 110) (end 110 110) (stroke (width 0.05) (type default)) (layer "Edge.Cuts"))
 (gr_line (start 120 25) (end 130 25) (stroke (width 0.05) (type default)) (layer "Edge.Cuts"))
 (gr_line (start 120 35) (end 120 25) (stroke (width 0.05) (type default)) (layer "Edge.Cuts"))
 (gr_line (start 120 105) (end 115 105) (stroke (width 0.05) (type default)) (layer "Edge.Cuts"))
 (gr_line (start 120 110) (end 120 105) (stroke (width 0.05) (type default)) (layer "Edge.Cuts"))
 (gr_line (start 125 110) (end 120 110) (stroke (width 0.05) (type default)) (layer "Edge.Cuts"))
 (gr_line (start 125 115) (end 125 110) (stroke (width 0.05) (type default)) (layer "Edge.Cuts"))
 (gr_line (start 130 25) (end 130 35) (stroke (width 0.05) (type default)) (layer "Edge.Cuts"))
 (gr_line (start 130 35) (end 135 35) (stroke (width 0.05) (type default)) (layer "Edge.Cuts"))
 (gr_line (start 130 115) (end 125 115) (stroke (width 0.05) (type default)) (layer "Edge.Cuts"))
 (gr_line (start 130 120.5) (end 130 115) (stroke (width 0.05) (type default)) (layer "Edge.Cuts"))
 (gr_line (start 135 35) (end 135 45) (stroke (width 0.05) (type default)) (layer "Edge.Cuts"))
 (gr_line (start 135 45) (end 140 45) (stroke (width 0.05) (type default)) (layer "Edge.Cuts"))
 (gr_line (start 135 120.5) (end 130 120.5) (stroke (width 0.05) (type default)) (layer "Edge.Cuts"))
 (gr_line (start 135 124.5) (end 135 120.5) (stroke (width 0.05) (type default)) (layer "Edge.Cuts"))
 (gr_line (start 140 45) (end 140 55) (stroke (width 0.05) (type default)) (layer "Edge.Cuts"))
 (gr_line (start 140 55) (end 145 55) (stroke (width 0.05) (type default)) (layer "Edge.Cuts"))
 (gr_line (start 145 55) (end 145 60.5) (stroke (width 0.05) (type default)) (layer "Edge.Cuts"))
 (gr_line (start 145 60.5) (end 150 60.5) (stroke (width 0.05) (type default)) (layer "Edge.Cuts"))
 (gr_line (start 145 124.5) (end 135 124.5) (stroke (width 0.05) (type default)) (layer "Edge.Cuts"))
 (gr_line (start 145 130) (end 145 124.5) (stroke (width 0.05) (type default)) (layer "Edge.Cuts"))
 (gr_line (start 150 60.5) (end 150 65) (stroke (width 0.05) (type default)) (layer "Edge.Cuts"))
 (gr_line (start 150 65) (end 180 65) (stroke (width 0.05) (type default)) (layer "Edge.Cuts"))
 (gr_line (start 150 100.5) (end 150 105) (stroke (width 0.05) (type default)) (layer "Edge.Cuts"))
 (gr_line (start 150 105) (end 155 105) (stroke (width 0.05) (type default)) (layer "Edge.Cuts"))
 (gr_line (start 150 130) (end 145 130) (stroke (width 0.05) (type default)) (layer "Edge.Cuts"))
 (gr_line (start 150 135.5) (end 150 130) (stroke (width 0.05) (type default)) (layer "Edge.Cuts"))
 (gr_line (start 155 95) (end 155 100.5) (stroke (width 0.05) (type default)) (layer "Edge.Cuts"))
 (gr_line (start 155 100.5) (end 150 100.5) (stroke (width 0.05) (type default)) (layer "Edge.Cuts"))
 (gr_line (start 155 105) (end 155 115) (stroke (width 0.05) (type default)) (layer "Edge.Cuts"))
 (gr_line (start 155 115) (end 160 115) (stroke (width 0.05) (type default)) (layer "Edge.Cuts"))
 (gr_line (start 159.5 85) (end 159.5 95) (stroke (width 0.05) (type default)) (layer "Edge.Cuts"))
 (gr_line (start 159.5 95) (end 155 95) (stroke (width 0.05) (type default)) (layer "Edge.Cuts"))
 (gr_line (start 160 115) (end 160 124.5) (stroke (width 0.05) (type default)) (layer "Edge.Cuts"))
 (gr_line (start 160 124.5) (end 165 124.5) (stroke (width 0.05) (type default)) (layer "Edge.Cuts"))
 (gr_line (start 165 80) (end 165 85) (stroke (width 0.05) (type default)) (layer "Edge.Cuts"))
 (gr_line (start 165 85) (end 159.5 85) (stroke (width 0.05) (type default)) (layer "Edge.Cuts"))
 (gr_line (start 165 124.5) (end 165 135.5) (stroke (width 0.05) (type default)) (layer "Edge.Cuts"))
 (gr_line (start 165 135.5) (end 150 135.5) (stroke (width 0.05) (type default)) (layer "Edge.Cuts"))
 (gr_line (start 170 75) (end 170 80) (stroke (width 0.05) (type default)) (layer "Edge.Cuts"))
 (gr_line (start 170 80) (end 165 80) (stroke (width 0.05) (type default)) (layer "Edge.Cuts"))
 (gr_line (start 175 70) (end 175 75) (stroke (width 0.05) (type default)) (layer "Edge.Cuts"))
 (gr_line (start 175 75) (end 170 75) (stroke (width 0.05) (type default)) (layer "Edge.Cuts"))
 (gr_line (start 180 65) (end 180 70) (stroke (width 0.05) (type default)) (layer "Edge.Cuts"))
 (gr_line (start 180 70) (end 175 70) (stroke (width 0.05) (type default)) (layer "Edge.Cuts"))
 (segment (start 118.55 57.55) (end 117.5 56.5) (width 0.2) (layer "F.Cu") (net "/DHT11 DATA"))
 (segment (start 121.09 57.55) (end 118.55 57.55) (width 0.2) (layer "F.Cu") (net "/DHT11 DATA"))
 (segment (start 131.5 72) (end 131 72) (width 0.2) (layer "F.Cu") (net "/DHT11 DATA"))
 (segment (start 117.5 58.5) (end 117.5 56.5) (width 0.2) (layer "F.Cu") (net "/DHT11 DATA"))
 (segment (start 121.09 52.67) (end 121.09 57.55) (width 0.2) (layer "F.Cu") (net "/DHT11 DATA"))
 (segment (start 131.302 71.802) (end 131.5 72) (width 0.2) (layer "F.Cu") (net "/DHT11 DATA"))
 (segment (start 119.92 51.5) (end 121.09 52.67) (width 0.2) (layer "F.Cu") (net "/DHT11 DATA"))
 (segment (start 130.89 71.802) (end 131.302 71.802) (width 0.2) (layer "F.Cu") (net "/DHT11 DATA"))
 (segment (start 131 72) (end 117.5 58.5) (width 0.2) (layer "F.Cu") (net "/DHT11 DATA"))
 (segment (start 93.35 69.46) (end 98.232 74.342) (width 0.2) (layer "F.Cu") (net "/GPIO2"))
 (segment (start 98.232 74.342) (end 130.89 74.342) (width 0.2) (layer "F.Cu") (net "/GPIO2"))
 (segment (start 121.618 76.882) (end 104.5 94) (width 0.2) (layer "F.Cu") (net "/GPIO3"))
 (segment (start 130.89 76.882) (end 121.618 76.882) (width 0.2) (layer "F.Cu") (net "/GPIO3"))
 (segment (start 127.5 99.46) (end 123.44 95.4) (width 0.2) (layer "F.Cu") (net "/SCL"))
 (segment (start 91.95 68.880101) (end 95.730101 65.1) (width 0.2) (layer "F.Cu") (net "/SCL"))
 (segment (start 93.929899 72.019798) (end 91.95 70.039899) (width 0.2) (layer "F.Cu") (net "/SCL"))
 (segment (start 111.662 65.1) (end 115.27 61.492) (width 0.2) (layer "F.Cu") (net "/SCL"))
 (segment (start 91.95 70.039899) (end 91.95 68.880101) (width 0.2) (layer "F.Cu") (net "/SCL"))
 (segment (start 123.44 95.4) (end 103.920101 95.4) (width 0.2) (layer "F.Cu") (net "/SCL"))
 (segment (start 95.730101 65.1) (end 111.662 65.1) (width 0.2) (layer "F.Cu") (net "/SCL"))
 (segment (start 93.929899 85.409798) (end 93.929899 72.019798) (width 0.2) (layer "F.Cu") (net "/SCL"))
 (segment (start 103.920101 95.4) (end 93.929899 85.409798) (width 0.2) (layer "F.Cu") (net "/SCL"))
 (segment (start 132.565 68.423358) (end 132.565 96.935) (width 0.2) (layer "F.Cu") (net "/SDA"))
 (segment (start 132.103642 67.962) (end 132.565 68.423358) (width 0.2) (layer "F.Cu") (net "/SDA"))
 (segment (start 127.5 102) (end 129.215 100.285) (width 0.2) (layer "F.Cu") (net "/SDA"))
 (segment (start 129.215 83.637) (end 130.89 81.962) (width 0.2) (layer "F.Cu") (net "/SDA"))
 (segment (start 112.714214 52.5) (end 111.885786 52.5) (width 0.2) (layer "F.Cu") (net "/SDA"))
 (segment (start 129.215 100.285) (end 129.215 83.637) (width 0.2) (layer "F.Cu") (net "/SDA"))
 (segment (start 111.885786 52.5) (end 111.3 51.914214) (width 0.2) (layer "F.Cu") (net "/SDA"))
 (segment (start 132.565 96.935) (end 127.5 102) (width 0.2) (layer "F.Cu") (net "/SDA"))
 (segment (start 111.3 51.914214) (end 111.3 51.085786) (width 0.2) (layer "F.Cu") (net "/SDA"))
 (segment (start 111.3 51.085786) (end 111.885786 50.5) (width 0.2) (layer "F.Cu") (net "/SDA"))
 (segment (start 121.49 51.655786) (end 121.49 61.924314) (width 0.2) (layer "F.Cu") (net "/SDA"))
 (segment (start 120.334214 50.5) (end 121.49 51.655786) (width 0.2) (layer "F.Cu") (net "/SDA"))
 (segment (start 127.527686 67.962) (end 132.103642 67.962) (width 0.2) (layer "F.Cu") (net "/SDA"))
 (segment (start 117.81 61.492) (end 116.45 60.132) (width 0.2) (layer "F.Cu") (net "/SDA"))
 (segment (start 121.49 61.924314) (end 127.527686 67.962) (width 0.2) (layer "F.Cu") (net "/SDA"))
 (segment (start 111.885786 50.5) (end 120.334214 50.5) (width 0.2) (layer "F.Cu") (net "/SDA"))
 (segment (start 116.45 56.235786) (end 112.714214 52.5) (width 0.2) (layer "F.Cu") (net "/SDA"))
 (segment (start 116.45 60.132) (end 116.45 56.235786) (width 0.2) (layer "F.Cu") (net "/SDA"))
 (segment (start 115.04 51.5) (end 120.04 56.5) (width 0.2) (layer "F.Cu") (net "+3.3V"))
 (segment (start 112.3 51.5) (end 115.04 51.5) (width 0.2) (layer "F.Cu") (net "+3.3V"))
 (segment (start 112.73 61.492) (end 113.88 60.342) (width 0.2) (layer "B.Cu") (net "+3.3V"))
 (segment (start 147 84.5) (end 137.12 94.38) (width 0.2) (layer "B.Cu") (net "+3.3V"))
 (segment (start 113.88 60.342) (end 116.198 60.342) (width 0.2) (layer "B.Cu") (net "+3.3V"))
 (segment (start 137.12 94.38) (end 127.5 94.38) (width 0.2) (layer "B.Cu") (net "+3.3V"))
 (segment (start 116.198 60.342) (end 120.04 56.5) (width 0.2) (layer "B.Cu") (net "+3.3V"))
 (segment (start 147 74.5) (end 147 84.5) (width 0.2) (layer "B.Cu") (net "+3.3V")))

